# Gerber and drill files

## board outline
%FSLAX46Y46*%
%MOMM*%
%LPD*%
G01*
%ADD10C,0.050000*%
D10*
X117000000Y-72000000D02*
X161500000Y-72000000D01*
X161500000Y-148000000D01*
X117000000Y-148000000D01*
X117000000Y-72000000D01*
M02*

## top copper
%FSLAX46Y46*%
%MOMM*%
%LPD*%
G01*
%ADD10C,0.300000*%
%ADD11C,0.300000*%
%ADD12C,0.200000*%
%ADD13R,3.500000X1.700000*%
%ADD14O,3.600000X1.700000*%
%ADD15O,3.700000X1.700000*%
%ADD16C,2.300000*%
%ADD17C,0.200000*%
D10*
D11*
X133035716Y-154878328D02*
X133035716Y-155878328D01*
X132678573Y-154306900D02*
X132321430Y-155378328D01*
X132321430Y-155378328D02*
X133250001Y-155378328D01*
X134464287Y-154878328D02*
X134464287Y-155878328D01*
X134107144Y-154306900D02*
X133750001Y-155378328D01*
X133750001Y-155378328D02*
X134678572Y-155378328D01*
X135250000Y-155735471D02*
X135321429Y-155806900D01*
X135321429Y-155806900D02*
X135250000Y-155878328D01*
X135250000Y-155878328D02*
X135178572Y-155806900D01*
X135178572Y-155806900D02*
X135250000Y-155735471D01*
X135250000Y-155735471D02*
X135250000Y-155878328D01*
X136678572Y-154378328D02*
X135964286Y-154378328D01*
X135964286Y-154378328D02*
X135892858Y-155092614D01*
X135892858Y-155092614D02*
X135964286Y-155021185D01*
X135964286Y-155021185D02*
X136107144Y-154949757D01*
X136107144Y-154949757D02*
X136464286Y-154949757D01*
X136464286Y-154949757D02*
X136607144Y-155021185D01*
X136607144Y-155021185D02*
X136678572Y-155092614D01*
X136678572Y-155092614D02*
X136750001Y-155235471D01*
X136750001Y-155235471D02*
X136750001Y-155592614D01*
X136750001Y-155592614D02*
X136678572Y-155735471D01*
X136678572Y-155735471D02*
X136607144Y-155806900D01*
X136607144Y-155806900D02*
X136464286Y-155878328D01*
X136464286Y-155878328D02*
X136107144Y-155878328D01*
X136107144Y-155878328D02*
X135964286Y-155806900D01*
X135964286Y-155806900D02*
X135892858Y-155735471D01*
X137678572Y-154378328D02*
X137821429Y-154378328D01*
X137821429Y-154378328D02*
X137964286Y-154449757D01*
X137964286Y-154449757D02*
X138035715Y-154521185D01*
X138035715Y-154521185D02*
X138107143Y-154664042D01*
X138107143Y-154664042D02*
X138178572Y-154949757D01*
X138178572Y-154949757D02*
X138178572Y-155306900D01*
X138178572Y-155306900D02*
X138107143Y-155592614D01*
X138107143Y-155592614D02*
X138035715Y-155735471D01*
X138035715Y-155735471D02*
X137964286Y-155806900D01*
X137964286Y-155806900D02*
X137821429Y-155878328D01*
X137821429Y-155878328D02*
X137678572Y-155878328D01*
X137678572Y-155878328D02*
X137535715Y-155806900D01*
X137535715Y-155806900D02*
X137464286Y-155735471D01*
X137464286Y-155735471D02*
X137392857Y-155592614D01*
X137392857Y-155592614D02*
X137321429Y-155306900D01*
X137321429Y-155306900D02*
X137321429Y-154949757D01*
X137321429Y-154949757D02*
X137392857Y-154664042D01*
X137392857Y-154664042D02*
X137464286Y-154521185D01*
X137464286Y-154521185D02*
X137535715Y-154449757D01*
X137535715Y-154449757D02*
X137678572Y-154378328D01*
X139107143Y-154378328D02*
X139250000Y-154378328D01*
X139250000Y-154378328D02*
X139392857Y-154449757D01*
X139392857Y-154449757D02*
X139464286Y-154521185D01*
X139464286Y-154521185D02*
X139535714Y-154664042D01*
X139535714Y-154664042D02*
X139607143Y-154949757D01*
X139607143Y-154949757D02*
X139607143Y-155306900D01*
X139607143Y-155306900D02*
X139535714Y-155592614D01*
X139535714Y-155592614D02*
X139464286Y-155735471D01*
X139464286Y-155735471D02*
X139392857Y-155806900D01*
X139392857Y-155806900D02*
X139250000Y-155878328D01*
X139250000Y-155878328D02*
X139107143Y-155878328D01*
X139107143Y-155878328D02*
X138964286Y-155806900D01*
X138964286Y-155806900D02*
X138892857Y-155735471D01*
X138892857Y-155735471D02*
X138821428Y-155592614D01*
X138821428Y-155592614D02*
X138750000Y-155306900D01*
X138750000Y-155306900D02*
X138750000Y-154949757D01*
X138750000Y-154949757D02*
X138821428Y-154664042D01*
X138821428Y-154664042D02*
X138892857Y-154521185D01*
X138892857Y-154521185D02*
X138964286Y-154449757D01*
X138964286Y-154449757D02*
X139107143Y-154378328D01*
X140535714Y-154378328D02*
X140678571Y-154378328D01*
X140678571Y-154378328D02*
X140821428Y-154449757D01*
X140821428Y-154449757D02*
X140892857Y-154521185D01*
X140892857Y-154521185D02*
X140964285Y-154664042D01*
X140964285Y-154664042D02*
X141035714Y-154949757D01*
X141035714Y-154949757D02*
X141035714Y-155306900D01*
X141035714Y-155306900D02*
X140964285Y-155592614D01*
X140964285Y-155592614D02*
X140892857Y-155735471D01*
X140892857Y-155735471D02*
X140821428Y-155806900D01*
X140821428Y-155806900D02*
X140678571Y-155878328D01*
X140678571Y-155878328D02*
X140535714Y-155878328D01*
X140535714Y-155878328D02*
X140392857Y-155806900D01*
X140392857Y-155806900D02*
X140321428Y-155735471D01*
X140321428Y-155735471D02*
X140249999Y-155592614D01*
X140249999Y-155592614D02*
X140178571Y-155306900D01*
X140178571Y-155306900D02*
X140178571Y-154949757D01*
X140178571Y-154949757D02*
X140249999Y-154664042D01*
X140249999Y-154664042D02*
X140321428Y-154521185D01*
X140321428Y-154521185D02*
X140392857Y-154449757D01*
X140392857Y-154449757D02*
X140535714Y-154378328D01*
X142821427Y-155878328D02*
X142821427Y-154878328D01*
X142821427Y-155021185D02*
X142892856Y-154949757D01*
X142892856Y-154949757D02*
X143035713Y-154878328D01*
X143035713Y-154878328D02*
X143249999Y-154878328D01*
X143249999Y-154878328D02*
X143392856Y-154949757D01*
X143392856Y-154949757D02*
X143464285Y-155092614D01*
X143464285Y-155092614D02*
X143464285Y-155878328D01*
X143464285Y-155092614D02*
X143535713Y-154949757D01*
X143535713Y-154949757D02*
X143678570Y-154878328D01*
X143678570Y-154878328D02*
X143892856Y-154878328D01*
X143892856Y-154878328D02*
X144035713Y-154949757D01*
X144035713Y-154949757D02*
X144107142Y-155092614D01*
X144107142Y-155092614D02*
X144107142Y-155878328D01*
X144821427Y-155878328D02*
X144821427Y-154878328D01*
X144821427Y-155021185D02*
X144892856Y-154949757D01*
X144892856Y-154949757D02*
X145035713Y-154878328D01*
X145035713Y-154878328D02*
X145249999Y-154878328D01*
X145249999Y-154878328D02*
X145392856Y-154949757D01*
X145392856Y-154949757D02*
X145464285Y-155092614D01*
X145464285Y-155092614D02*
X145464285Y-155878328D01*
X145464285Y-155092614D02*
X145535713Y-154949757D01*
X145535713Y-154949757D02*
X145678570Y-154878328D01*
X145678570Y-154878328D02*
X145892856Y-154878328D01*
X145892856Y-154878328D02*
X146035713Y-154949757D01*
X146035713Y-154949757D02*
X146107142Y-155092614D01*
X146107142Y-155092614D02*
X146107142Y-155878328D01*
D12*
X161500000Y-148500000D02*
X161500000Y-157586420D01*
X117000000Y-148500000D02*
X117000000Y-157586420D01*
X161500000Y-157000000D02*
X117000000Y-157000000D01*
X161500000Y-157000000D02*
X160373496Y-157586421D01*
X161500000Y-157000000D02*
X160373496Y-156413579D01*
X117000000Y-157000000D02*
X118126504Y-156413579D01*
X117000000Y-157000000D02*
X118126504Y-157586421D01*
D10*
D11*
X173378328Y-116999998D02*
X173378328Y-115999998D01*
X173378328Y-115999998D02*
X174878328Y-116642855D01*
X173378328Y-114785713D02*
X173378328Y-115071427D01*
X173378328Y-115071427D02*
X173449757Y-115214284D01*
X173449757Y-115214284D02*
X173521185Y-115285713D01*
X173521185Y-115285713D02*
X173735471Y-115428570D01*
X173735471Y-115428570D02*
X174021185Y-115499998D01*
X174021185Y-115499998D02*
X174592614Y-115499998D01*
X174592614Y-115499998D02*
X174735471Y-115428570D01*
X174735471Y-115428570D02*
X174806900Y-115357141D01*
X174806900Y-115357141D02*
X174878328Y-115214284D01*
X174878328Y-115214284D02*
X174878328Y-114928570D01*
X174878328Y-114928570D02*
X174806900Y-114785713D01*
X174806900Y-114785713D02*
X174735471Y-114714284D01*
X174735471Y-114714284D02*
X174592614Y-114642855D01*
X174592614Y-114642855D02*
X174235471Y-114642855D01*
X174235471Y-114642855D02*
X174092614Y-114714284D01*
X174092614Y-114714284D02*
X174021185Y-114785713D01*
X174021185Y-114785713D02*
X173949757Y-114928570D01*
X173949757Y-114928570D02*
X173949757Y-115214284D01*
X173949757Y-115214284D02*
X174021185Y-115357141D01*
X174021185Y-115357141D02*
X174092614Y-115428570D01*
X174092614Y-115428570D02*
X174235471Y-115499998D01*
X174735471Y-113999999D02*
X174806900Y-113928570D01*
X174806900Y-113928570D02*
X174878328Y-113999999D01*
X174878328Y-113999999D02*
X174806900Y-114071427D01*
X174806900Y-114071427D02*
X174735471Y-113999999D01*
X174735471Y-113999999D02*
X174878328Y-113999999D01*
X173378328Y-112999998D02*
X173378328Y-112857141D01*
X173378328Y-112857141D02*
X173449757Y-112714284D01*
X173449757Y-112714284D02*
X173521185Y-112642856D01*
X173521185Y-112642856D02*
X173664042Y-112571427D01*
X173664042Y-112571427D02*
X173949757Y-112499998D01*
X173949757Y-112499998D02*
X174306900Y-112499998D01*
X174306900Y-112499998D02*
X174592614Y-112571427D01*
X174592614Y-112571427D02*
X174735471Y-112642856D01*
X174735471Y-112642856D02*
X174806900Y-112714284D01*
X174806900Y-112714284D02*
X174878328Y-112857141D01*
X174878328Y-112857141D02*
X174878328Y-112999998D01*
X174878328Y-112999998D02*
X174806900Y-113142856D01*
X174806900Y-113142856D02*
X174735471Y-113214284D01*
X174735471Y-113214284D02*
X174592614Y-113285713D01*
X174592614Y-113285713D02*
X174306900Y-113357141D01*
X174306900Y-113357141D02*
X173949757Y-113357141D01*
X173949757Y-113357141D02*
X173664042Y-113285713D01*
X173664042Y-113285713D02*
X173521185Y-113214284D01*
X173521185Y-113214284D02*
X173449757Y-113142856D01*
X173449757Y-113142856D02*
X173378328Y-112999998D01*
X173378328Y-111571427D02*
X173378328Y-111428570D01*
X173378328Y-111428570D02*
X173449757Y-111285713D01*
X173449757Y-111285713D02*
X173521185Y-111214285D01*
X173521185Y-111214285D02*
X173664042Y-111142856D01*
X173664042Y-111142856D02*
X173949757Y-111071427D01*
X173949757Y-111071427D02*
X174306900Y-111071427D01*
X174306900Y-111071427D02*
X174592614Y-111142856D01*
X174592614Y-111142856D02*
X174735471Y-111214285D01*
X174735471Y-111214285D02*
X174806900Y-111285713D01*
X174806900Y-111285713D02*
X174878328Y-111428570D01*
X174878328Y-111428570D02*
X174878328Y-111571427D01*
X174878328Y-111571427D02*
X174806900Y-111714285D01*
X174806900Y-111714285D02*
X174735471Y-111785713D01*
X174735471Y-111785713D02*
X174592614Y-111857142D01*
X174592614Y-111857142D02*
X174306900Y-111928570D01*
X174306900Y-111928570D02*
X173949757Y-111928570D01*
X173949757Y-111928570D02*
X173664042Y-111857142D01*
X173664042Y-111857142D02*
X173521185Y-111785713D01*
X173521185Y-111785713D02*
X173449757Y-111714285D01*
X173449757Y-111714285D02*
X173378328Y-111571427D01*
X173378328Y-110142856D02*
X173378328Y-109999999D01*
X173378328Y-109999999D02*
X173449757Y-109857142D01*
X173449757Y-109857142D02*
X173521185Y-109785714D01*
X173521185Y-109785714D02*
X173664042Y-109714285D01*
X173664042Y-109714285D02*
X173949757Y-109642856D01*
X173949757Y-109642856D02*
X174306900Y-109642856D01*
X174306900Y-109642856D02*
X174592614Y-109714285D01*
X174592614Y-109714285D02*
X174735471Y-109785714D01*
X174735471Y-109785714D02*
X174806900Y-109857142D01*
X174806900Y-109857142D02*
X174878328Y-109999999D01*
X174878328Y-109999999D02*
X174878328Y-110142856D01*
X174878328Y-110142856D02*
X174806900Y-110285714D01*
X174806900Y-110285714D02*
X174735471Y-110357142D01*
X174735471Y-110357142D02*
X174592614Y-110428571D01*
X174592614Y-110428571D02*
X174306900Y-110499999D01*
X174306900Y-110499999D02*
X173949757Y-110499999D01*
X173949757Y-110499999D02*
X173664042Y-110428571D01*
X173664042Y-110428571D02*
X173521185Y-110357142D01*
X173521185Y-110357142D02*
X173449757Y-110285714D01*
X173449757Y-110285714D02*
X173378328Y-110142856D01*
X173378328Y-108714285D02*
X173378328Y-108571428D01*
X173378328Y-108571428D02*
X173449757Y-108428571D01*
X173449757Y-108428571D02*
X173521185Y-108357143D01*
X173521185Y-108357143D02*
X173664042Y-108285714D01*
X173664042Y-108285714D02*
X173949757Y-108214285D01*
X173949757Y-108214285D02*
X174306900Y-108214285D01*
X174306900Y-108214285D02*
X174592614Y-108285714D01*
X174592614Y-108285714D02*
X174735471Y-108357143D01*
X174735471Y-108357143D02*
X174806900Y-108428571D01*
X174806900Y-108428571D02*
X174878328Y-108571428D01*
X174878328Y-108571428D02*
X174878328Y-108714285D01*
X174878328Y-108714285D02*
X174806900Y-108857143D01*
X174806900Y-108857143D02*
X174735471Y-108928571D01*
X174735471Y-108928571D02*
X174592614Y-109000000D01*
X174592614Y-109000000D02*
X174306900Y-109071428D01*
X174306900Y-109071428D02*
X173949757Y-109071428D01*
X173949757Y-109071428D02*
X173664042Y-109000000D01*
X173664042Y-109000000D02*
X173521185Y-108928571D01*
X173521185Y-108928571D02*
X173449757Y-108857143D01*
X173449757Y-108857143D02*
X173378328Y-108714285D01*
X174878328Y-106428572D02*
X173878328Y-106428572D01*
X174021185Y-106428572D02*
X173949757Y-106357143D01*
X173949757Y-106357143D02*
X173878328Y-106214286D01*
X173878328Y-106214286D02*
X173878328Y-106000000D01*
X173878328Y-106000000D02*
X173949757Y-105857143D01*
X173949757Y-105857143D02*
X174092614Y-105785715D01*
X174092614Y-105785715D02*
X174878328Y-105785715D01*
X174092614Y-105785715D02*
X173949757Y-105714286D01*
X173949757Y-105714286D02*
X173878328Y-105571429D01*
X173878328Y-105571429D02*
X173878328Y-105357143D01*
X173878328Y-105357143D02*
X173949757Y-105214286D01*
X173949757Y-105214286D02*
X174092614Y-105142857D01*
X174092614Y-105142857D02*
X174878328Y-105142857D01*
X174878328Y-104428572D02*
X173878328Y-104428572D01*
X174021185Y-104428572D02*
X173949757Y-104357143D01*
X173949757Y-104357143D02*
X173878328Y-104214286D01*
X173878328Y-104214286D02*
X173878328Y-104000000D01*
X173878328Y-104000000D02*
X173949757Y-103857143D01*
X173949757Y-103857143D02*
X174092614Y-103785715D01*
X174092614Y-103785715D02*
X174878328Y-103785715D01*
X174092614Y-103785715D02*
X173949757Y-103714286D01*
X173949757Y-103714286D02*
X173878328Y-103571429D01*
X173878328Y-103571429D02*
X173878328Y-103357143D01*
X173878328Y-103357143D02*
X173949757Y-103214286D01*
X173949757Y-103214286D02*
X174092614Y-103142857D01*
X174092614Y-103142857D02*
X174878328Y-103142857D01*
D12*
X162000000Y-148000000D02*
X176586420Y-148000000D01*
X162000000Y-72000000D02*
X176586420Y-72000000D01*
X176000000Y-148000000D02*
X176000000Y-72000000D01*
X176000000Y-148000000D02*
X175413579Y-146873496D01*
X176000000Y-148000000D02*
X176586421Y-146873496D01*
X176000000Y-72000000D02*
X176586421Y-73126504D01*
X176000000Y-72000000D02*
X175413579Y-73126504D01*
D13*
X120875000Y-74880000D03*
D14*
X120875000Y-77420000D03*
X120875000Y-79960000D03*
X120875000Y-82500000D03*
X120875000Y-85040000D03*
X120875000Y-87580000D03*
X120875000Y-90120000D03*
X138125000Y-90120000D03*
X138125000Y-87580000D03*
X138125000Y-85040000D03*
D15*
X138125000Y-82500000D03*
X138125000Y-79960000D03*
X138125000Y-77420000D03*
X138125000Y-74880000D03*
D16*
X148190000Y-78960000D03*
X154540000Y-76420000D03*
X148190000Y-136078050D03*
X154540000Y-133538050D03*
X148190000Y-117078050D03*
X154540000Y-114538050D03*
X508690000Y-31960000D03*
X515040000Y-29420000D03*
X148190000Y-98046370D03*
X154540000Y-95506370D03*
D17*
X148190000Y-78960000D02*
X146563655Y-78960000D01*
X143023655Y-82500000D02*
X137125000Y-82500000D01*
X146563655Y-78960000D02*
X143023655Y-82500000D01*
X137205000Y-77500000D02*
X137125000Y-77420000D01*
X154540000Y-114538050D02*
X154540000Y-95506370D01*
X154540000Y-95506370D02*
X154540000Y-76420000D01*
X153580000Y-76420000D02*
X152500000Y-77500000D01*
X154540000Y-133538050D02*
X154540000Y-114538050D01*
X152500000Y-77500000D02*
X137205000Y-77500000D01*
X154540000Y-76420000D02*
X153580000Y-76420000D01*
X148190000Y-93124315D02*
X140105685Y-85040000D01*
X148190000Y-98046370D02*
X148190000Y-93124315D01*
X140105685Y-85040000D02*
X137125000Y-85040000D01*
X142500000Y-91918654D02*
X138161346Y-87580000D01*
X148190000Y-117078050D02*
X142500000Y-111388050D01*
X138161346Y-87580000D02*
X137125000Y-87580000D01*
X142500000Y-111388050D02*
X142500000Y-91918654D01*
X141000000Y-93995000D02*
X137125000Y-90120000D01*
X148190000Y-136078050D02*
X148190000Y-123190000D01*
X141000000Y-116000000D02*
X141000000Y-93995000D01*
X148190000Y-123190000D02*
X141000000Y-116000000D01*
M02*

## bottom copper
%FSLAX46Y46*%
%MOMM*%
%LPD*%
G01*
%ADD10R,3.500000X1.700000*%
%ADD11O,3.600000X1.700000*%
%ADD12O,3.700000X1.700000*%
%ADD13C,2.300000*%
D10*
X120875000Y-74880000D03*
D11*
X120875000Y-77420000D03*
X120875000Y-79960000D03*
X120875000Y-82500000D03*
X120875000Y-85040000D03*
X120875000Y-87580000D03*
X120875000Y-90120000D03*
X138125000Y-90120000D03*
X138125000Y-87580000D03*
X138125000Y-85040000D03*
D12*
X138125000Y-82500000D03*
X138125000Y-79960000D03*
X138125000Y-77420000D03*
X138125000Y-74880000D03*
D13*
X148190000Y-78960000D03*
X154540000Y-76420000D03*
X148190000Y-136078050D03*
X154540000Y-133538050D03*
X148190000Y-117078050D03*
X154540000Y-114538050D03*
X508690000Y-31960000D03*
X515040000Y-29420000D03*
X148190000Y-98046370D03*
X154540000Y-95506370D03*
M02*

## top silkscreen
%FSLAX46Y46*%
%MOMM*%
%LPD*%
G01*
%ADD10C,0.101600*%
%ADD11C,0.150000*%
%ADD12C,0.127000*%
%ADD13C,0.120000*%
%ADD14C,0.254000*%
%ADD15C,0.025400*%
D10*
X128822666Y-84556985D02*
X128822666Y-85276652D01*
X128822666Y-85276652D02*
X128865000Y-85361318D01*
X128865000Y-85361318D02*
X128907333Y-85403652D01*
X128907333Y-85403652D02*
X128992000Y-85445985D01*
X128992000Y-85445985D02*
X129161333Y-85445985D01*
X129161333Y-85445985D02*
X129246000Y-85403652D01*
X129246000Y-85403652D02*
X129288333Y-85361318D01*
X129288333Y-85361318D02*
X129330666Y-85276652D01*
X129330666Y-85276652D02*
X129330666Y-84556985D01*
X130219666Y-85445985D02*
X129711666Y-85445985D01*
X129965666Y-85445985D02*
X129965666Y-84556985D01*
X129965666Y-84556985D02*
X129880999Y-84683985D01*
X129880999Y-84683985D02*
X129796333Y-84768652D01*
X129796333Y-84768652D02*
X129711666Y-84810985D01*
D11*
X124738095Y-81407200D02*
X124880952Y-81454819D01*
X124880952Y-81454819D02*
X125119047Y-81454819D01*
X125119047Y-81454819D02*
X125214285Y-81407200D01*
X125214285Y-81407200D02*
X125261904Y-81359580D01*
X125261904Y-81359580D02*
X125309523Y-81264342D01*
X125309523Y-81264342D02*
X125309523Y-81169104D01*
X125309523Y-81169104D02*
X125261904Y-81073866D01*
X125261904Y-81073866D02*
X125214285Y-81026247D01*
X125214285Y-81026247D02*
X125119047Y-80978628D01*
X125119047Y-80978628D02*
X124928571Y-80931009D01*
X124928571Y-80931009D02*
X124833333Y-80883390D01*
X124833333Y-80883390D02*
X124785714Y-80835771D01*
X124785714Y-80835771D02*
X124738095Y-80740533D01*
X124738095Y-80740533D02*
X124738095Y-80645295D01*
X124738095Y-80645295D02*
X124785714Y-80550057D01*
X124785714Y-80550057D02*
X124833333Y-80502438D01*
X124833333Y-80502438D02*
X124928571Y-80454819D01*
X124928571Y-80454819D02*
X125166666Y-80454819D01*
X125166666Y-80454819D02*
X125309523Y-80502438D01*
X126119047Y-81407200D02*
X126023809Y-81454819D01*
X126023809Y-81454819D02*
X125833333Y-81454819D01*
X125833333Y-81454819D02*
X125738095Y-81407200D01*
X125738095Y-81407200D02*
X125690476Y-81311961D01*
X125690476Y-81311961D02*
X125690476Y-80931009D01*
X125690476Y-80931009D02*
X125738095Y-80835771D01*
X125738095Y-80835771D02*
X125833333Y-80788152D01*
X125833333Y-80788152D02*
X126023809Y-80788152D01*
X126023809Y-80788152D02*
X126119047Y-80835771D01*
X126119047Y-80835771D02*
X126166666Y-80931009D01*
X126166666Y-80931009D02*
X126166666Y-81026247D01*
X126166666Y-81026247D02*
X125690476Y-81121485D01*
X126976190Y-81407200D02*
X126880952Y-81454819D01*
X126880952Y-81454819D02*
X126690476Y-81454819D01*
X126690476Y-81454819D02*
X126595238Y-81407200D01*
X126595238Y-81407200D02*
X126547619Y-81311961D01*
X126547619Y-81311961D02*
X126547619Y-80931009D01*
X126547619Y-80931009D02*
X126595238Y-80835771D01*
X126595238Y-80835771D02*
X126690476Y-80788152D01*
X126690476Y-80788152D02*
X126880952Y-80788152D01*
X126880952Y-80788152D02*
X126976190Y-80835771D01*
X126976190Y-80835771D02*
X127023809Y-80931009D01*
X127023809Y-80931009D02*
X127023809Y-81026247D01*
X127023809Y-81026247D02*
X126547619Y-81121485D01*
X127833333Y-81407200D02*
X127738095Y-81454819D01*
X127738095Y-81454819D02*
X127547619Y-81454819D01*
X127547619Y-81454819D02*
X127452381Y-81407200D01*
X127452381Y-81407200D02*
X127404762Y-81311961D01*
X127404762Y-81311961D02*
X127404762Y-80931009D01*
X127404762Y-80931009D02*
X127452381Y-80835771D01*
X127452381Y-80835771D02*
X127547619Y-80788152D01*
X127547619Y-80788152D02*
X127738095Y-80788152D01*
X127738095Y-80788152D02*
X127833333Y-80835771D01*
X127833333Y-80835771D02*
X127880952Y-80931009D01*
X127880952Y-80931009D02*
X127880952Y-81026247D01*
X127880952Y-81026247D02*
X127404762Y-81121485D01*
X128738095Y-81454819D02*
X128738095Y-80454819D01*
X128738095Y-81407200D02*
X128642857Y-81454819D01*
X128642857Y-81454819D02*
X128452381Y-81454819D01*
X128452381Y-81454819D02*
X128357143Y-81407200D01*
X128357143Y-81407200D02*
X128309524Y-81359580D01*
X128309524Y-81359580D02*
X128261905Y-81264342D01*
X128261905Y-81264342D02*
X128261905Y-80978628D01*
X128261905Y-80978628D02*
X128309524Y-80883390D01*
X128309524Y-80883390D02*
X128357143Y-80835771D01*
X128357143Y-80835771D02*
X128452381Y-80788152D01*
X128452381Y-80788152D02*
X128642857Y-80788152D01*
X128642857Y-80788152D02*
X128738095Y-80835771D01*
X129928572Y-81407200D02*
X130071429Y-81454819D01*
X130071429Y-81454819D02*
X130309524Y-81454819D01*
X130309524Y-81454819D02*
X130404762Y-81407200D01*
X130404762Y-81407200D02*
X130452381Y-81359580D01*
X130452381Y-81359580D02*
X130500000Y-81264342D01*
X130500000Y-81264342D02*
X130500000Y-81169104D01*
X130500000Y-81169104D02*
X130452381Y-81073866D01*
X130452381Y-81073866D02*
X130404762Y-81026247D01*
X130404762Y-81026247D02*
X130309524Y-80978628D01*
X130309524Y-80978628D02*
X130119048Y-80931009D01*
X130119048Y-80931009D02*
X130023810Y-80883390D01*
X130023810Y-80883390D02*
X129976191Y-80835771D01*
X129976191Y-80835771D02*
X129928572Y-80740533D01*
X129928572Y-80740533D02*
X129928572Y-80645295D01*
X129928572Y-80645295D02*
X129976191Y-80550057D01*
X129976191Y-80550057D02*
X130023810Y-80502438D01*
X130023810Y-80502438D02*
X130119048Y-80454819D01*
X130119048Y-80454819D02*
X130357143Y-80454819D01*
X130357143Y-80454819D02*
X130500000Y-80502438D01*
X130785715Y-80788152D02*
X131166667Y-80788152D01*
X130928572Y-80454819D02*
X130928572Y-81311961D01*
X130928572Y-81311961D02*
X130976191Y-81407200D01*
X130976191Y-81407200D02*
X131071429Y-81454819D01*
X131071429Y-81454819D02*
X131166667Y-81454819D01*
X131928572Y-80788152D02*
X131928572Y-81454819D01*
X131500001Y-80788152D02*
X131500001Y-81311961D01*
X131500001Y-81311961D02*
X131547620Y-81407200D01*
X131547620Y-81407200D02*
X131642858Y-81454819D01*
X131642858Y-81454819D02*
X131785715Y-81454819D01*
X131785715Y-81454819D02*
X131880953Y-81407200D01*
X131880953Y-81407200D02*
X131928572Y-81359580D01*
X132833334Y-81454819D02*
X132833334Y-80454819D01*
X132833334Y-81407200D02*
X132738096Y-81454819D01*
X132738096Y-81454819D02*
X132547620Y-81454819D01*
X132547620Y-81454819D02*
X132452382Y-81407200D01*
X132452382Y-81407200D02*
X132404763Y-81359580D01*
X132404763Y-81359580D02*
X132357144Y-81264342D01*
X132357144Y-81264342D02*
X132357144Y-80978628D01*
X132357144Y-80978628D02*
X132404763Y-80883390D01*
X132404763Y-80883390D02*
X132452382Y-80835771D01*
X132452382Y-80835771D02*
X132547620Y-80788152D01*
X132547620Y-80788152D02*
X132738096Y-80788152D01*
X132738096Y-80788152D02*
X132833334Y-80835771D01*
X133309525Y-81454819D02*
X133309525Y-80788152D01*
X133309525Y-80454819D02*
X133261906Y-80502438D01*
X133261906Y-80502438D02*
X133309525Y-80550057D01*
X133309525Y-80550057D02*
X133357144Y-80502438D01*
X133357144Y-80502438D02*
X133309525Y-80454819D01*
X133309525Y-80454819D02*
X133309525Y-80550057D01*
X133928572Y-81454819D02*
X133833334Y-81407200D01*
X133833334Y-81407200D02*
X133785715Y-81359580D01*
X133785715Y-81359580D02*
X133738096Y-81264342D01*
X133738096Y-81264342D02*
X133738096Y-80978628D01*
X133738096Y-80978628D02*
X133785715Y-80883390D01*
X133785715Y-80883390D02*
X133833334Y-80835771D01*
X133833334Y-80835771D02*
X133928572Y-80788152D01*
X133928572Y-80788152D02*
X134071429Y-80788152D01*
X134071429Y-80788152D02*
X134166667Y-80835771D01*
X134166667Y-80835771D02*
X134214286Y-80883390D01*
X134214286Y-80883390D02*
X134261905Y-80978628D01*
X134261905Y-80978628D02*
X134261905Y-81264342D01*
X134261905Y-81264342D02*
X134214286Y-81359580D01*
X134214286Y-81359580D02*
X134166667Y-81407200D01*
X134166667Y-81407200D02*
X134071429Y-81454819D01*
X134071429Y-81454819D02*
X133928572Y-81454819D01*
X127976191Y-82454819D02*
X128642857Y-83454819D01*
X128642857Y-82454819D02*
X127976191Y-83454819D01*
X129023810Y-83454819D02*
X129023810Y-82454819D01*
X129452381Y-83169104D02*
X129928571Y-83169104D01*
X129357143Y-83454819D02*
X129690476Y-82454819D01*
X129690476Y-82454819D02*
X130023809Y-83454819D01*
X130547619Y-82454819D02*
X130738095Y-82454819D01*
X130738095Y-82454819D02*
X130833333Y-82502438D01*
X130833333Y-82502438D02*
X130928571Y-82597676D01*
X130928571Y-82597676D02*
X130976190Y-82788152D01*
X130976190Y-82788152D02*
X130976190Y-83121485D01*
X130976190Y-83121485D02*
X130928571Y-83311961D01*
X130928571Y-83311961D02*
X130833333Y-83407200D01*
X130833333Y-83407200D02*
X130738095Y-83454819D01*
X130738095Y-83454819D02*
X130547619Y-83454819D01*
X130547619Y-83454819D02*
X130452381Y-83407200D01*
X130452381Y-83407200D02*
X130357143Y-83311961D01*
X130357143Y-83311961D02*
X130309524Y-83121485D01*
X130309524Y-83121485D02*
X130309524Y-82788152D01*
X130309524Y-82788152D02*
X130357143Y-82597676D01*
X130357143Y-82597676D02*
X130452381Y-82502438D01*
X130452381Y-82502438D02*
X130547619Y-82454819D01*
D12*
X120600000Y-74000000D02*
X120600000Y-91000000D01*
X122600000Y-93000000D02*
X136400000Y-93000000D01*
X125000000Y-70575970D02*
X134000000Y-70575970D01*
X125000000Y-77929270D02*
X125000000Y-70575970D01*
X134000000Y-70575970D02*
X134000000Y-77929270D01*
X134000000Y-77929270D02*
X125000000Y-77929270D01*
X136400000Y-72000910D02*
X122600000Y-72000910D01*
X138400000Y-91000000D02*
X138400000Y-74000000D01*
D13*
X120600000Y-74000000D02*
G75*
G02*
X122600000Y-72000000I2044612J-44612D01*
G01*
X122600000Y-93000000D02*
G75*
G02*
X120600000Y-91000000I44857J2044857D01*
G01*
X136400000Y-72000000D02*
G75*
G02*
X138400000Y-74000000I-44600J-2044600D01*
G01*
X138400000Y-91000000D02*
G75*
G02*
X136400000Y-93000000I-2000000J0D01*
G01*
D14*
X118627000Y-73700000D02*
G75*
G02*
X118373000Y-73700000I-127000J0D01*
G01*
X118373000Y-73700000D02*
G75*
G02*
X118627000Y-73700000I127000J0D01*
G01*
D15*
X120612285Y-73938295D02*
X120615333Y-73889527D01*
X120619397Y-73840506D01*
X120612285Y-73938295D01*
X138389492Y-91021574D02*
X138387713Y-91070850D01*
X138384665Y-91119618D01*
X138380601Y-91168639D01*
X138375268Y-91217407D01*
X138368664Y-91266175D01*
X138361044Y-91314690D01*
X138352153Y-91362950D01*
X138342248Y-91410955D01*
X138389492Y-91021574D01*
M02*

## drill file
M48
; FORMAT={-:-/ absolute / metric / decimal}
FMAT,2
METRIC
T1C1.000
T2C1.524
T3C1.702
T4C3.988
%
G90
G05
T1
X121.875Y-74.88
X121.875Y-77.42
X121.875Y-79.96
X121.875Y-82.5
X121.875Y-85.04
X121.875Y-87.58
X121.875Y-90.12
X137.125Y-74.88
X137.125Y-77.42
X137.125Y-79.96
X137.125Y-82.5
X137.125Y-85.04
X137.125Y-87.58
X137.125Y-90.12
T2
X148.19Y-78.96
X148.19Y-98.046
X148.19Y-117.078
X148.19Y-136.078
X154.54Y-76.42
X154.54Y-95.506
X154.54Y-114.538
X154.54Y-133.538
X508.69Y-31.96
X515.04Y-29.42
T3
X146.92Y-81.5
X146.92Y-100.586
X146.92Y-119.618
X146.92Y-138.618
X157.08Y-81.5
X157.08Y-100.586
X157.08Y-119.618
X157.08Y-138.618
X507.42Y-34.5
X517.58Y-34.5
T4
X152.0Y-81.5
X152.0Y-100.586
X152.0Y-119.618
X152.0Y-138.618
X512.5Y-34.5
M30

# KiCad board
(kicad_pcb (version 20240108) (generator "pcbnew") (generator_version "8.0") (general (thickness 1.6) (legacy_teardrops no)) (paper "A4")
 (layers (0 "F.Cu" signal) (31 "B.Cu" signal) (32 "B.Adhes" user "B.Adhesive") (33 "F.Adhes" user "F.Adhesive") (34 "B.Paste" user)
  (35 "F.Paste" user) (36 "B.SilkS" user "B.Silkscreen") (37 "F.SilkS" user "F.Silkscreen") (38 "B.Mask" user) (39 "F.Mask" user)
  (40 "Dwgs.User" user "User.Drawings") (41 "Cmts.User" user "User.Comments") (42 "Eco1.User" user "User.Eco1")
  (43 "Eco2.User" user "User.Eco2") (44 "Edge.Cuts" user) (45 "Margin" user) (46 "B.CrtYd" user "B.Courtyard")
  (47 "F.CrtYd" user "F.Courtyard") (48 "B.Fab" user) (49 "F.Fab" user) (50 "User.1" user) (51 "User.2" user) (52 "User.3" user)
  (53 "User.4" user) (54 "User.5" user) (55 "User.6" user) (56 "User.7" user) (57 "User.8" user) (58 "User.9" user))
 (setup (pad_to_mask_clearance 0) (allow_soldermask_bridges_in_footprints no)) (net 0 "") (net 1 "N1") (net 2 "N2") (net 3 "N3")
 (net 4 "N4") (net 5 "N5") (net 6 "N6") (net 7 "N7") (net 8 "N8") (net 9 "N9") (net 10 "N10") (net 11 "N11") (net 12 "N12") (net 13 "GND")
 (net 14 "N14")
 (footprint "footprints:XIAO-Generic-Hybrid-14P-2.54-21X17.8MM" (layer "F.Cu") (at 129.5 82.5)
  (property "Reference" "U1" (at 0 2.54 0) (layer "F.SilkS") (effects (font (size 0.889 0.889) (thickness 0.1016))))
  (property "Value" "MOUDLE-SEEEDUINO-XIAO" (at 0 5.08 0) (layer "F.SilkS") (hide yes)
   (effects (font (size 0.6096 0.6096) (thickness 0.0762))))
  (fp_line (start -8.9 -8.5) (end -8.9 8.5) (stroke (width 0.127) (type solid)) (layer "F.SilkS"))
  (fp_line (start -6.9 10.5) (end 6.9 10.5) (stroke (width 0.127) (type solid)) (layer "F.SilkS"))
  (fp_line (start -4.5 -11.92403) (end 4.5 -11.92403) (stroke (width 0.127) (type solid)) (layer "F.SilkS"))
  (fp_line (start -4.5 -4.57073) (end -4.5 -11.92403) (stroke (width 0.127) (type solid)) (layer "F.SilkS"))
  (fp_line (start 4.5 -11.92403) (end 4.5 -4.57073) (stroke (width 0.127) (type solid)) (layer "F.SilkS"))
  (fp_line (start 4.5 -4.57073) (end -4.5 -4.57073) (stroke (width 0.127) (type solid)) (layer "F.SilkS"))
  (fp_line (start 6.9 -10.49909) (end -6.9 -10.49909) (stroke (width 0.127) (type solid)) (layer "F.SilkS"))
  (fp_line (start 8.9 8.5) (end 8.9 -8.5) (stroke (width 0.127) (type solid)) (layer "F.SilkS"))
  (fp_arc (start -8.9 -8.5) (mid -8.301491 -9.901491) (end -6.9 -10.5) (stroke (width 0.12) (type solid)) (layer "F.SilkS"))
  (fp_arc (start -6.9 10.5) (mid -8.301423 9.901423) (end -8.9 8.5) (stroke (width 0.12) (type solid)) (layer "F.SilkS"))
  (fp_arc (start 6.9 -10.5) (mid 8.301492 -9.901492) (end 8.9 -8.5) (stroke (width 0.12) (type solid)) (layer "F.SilkS"))
  (fp_arc (start 8.9 8.5) (mid 8.314214 9.914214) (end 6.9 10.5) (stroke (width 0.12) (type solid)) (layer "F.SilkS"))
  (fp_circle (center -11 -8.8) (end -11 -9.054) (stroke (width 0) (type solid)) (fill solid) (layer "F.SilkS"))
  (fp_poly
   (pts (xy -8.887715 -8.561705) (xy -8.884667 -8.610473) (xy -8.880603 -8.659494)) (stroke (width 0.0254) (type solid)) (fill none)
   (layer "F.SilkS"))
  (fp_poly
   (pts (xy 8.889492 8.521574) (xy 8.887713 8.57085) (xy 8.884665 8.619618) (xy 8.880601 8.668639) (xy 8.875268 8.717407)
    (xy 8.868664 8.766175) (xy 8.861044 8.81469) (xy 8.852153 8.86295) (xy 8.842248 8.910955))
   (stroke (width 0.0254) (type solid)) (fill none) (layer "F.SilkS"))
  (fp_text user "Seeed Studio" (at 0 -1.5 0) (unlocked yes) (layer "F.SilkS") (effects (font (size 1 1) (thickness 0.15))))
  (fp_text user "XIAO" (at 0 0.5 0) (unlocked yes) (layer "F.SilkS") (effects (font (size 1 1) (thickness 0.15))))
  (pad "1" thru_hole rect (at -7.625 -7.62) (size 3.5 1.7) (drill 1 (offset -1 0)) (layers "*.Cu" "*.Mask") (remove_unused_layers no)
   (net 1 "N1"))
  (pad "2" thru_hole oval (at -7.625 -5.08) (size 3.6 1.7) (drill 1 (offset -1 0)) (layers "*.Cu" "*.Mask") (remove_unused_layers no)
   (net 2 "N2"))
  (pad "3" thru_hole oval (at -7.625 -2.54) (size 3.6 1.7) (drill 1 (offset -1 0)) (layers "*.Cu" "*.Mask") (remove_unused_layers no)
   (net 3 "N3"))
  (pad "4" thru_hole oval (at -7.625 0) (size 3.6 1.7) (drill 1 (offset -1 0)) (layers "*.Cu" "*.Mask") (remove_unused_layers no)
   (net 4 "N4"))
  (pad "5" thru_hole oval (at -7.625 2.54) (size 3.6 1.7) (drill 1 (offset -1 0)) (layers "*.Cu" "*.Mask") (remove_unused_layers no)
   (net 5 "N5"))
  (pad "6" thru_hole oval (at -7.625 5.08 180) (size 3.6 1.7) (drill 1 (offset 1 0)) (layers "*.Cu" "*.Mask") (remove_unused_layers no)
   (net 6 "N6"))
  (pad "7" thru_hole oval (at -7.625 7.62) (size 3.6 1.7) (drill 1 (offset -1 0)) (layers "*.Cu" "*.Mask") (remove_unused_layers no)
   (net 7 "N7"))
  (pad "8" thru_hole oval (at 7.625 7.62) (size 3.6 1.7) (drill 1 (offset 1 0)) (layers "*.Cu" "*.Mask") (remove_unused_layers no)
   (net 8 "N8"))
  (pad "9" thru_hole oval (at 7.625 5.08) (size 3.6 1.7) (drill 1 (offset 1 0)) (layers "*.Cu" "*.Mask") (remove_unused_layers no)
   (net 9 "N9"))
  (pad "10" thru_hole oval (at 7.625 2.54) (size 3.6 1.7) (drill 1 (offset 1 0)) (layers "*.Cu" "*.Mask") (remove_unused_layers no)
   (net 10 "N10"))
  (pad "11" thru_hole oval (at 7.625 0) (size 3.7 1.7) (drill 1 (offset 1 0)) (layers "*.Cu" "*.Mask") (remove_unused_layers no)
   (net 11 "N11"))
  (pad "12" thru_hole oval (at 7.625 -2.54) (size 3.7 1.7) (drill 1 (offset 1 0)) (layers "*.Cu" "*.Mask") (remove_unused_layers no)
   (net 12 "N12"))
  (pad "13" thru_hole oval (at 7.625 -5.08) (size 3.7 1.7) (drill 1 (offset 1 0)) (layers "*.Cu" "*.Mask") (remove_unused_layers no)
   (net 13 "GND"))
  (pad "14" thru_hole oval (at 7.625 -7.62) (size 3.7 1.7) (drill 1 (offset 1 0)) (layers "*.Cu" "*.Mask") (remove_unused_layers no)
   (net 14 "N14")))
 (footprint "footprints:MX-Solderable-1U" (layer "F.Cu") (at 152 81.5)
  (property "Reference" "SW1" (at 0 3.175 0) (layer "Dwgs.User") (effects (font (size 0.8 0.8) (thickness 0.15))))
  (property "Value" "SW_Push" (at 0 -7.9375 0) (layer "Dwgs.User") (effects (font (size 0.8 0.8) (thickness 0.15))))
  (pad "" np_thru_hole circle (at -5.08 0 48.099) (size 1.7018 1.7018) (drill 1.7018) (layers "F&B.Cu" "*.Mask"))
  (pad "" np_thru_hole circle (at 0 0) (size 3.9878 3.9878) (drill 3.9878) (layers "*.Cu" "*.Mask"))
  (pad "" np_thru_hole circle (at 5.08 0 48.099) (size 1.7018 1.7018) (drill 1.7018) (layers "F&B.Cu" "*.Mask"))
  (pad "1" thru_hole circle (at -3.81 -2.54) (size 2.3 2.3) (drill 1.524) (layers "*.Cu" "B.Mask") (remove_unused_layers no) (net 11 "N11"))
  (pad "2" thru_hole circle (at 2.54 -5.08) (size 2.3 2.3) (drill 1.524) (layers "*.Cu" "B.Mask") (remove_unused_layers no) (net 13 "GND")))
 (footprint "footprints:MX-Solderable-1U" (layer "F.Cu") (at 152 138.61805)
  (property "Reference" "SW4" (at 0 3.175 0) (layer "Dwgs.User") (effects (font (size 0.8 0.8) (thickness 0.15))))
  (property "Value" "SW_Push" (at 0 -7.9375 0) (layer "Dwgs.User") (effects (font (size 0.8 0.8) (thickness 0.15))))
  (pad "" np_thru_hole circle (at -5.08 0 48.099) (size 1.7018 1.7018) (drill 1.7018) (layers "F&B.Cu" "*.Mask"))
  (pad "" np_thru_hole circle (at 0 0) (size 3.9878 3.9878) (drill 3.9878) (layers "*.Cu" "*.Mask"))
  (pad "" np_thru_hole circle (at 5.08 0 48.099) (size 1.7018 1.7018) (drill 1.7018) (layers "F&B.Cu" "*.Mask"))
  (pad "1" thru_hole circle (at -3.81 -2.54) (size 2.3 2.3) (drill 1.524) (layers "*.Cu" "B.Mask") (remove_unused_layers no) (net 8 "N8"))
  (pad "2" thru_hole circle (at 2.54 -5.08) (size 2.3 2.3) (drill 1.524) (layers "*.Cu" "B.Mask") (remove_unused_layers no) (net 13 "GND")))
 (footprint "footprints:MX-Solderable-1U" (layer "F.Cu") (at 152 119.61805)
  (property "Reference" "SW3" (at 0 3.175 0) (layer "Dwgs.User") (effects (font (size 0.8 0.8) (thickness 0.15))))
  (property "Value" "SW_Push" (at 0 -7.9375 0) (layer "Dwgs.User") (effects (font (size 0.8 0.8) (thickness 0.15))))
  (pad "" np_thru_hole circle (at -5.08 0 48.099) (size 1.7018 1.7018) (drill 1.7018) (layers "F&B.Cu" "*.Mask"))
  (pad "" np_thru_hole circle (at 0 0) (size 3.9878 3.9878) (drill 3.9878) (layers "*.Cu" "*.Mask"))
  (pad "" np_thru_hole circle (at 5.08 0 48.099) (size 1.7018 1.7018) (drill 1.7018) (layers "F&B.Cu" "*.Mask"))
  (pad "1" thru_hole circle (at -3.81 -2.54) (size 2.3 2.3) (drill 1.524) (layers "*.Cu" "B.Mask") (remove_unused_layers no) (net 9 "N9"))
  (pad "2" thru_hole circle (at 2.54 -5.08) (size 2.3 2.3) (drill 1.524) (layers "*.Cu" "B.Mask") (remove_unused_layers no) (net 13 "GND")))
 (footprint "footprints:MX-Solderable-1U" (layer "F.Cu") (at 512.5 34.5)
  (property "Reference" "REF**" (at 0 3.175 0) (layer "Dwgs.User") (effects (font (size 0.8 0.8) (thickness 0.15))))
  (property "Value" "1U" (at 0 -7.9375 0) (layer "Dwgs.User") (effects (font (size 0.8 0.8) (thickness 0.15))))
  (pad "" np_thru_hole circle (at -5.08 0 48.099) (size 1.7018 1.7018) (drill 1.7018) (layers "F&B.Cu" "*.Mask"))
  (pad "" np_thru_hole circle (at 0 0) (size 3.9878 3.9878) (drill 3.9878) (layers "*.Cu" "*.Mask"))
  (pad "" np_thru_hole circle (at 5.08 0 48.099) (size 1.7018 1.7018) (drill 1.7018) (layers "F&B.Cu" "*.Mask"))
  (pad "1" thru_hole circle (at -3.81 -2.54) (size 2.3 2.3) (drill 1.524) (layers "*.Cu" "B.Mask") (remove_unused_layers no))
  (pad "2" thru_hole circle (at 2.54 -5.08) (size 2.3 2.3) (drill 1.524) (layers "*.Cu" "B.Mask") (remove_unused_layers no)))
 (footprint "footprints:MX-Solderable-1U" (layer "F.Cu") (at 152 100.58637)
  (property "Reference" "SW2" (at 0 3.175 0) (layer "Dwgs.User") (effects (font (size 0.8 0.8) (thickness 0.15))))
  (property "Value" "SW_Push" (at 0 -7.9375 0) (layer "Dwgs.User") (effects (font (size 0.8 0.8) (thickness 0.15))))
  (pad "" np_thru_hole circle (at -5.08 0 48.099) (size 1.7018 1.7018) (drill 1.7018) (layers "F&B.Cu" "*.Mask"))
  (pad "" np_thru_hole circle (at 0 0) (size 3.9878 3.9878) (drill 3.9878) (layers "*.Cu" "*.Mask"))
  (pad "" np_thru_hole circle (at 5.08 0 48.099) (size 1.7018 1.7018) (drill 1.7018) (layers "F&B.Cu" "*.Mask"))
  (pad "1" thru_hole circle (at -3.81 -2.54) (size 2.3 2.3) (drill 1.524) (layers "*.Cu" "B.Mask") (remove_unused_layers no) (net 10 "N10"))
  (pad "2" thru_hole circle (at 2.54 -5.08) (size 2.3 2.3) (drill 1.524) (layers "*.Cu" "B.Mask") (remove_unused_layers no) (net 13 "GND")))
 (gr_rect (start 117 72) (end 161.5 148) (stroke (width 0.05) (type default)) (fill none) (layer "Edge.Cuts"))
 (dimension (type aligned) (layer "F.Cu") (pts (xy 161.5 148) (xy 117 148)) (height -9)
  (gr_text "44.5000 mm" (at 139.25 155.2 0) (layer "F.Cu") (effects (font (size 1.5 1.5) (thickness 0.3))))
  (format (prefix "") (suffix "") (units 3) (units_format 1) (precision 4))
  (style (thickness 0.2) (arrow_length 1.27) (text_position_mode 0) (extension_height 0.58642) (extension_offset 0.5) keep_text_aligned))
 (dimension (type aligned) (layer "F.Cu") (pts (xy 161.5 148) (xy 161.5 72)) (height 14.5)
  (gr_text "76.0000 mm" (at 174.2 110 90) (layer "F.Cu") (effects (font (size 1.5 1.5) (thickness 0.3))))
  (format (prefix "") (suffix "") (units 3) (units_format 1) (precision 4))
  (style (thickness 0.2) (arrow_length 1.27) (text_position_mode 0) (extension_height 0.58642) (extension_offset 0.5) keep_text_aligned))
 (segment (start 148.19 78.96) (end 146.563655 78.96) (width 0.2) (layer "F.Cu") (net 11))
 (segment (start 143.023655 82.5) (end 137.125 82.5) (width 0.2) (layer "F.Cu") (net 11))
 (segment (start 146.563655 78.96) (end 143.023655 82.5) (width 0.2) (layer "F.Cu") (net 11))
 (segment (start 137.205 77.5) (end 137.125 77.42) (width 0.2) (layer "F.Cu") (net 13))
 (segment (start 154.54 114.53805) (end 154.54 95.50637) (width 0.2) (layer "F.Cu") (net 13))
 (segment (start 154.54 95.50637) (end 154.54 76.42) (width 0.2) (layer "F.Cu") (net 13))
 (segment (start 153.58 76.42) (end 152.5 77.5) (width 0.2) (layer "F.Cu") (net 13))
 (segment (start 154.54 133.53805) (end 154.54 114.53805) (width 0.2) (layer "F.Cu") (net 13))
 (segment (start 152.5 77.5) (end 137.205 77.5) (width 0.2) (layer "F.Cu") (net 13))
 (segment (start 154.54 76.42) (end 153.58 76.42) (width 0.2) (layer "F.Cu") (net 13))
 (segment (start 148.19 93.124315) (end 140.105685 85.04) (width 0.2) (layer "F.Cu") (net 10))
 (segment (start 148.19 98.04637) (end 148.19 93.124315) (width 0.2) (layer "F.Cu") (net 10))
 (segment (start 140.105685 85.04) (end 137.125 85.04) (width 0.2) (layer "F.Cu") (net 10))
 (segment (start 142.5 91.918654) (end 138.161346 87.58) (width 0.2) (layer "F.Cu") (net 9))
 (segment (start 148.19 117.07805) (end 142.5 111.38805) (width 0.2) (layer "F.Cu") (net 9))
 (segment (start 138.161346 87.58) (end 137.125 87.58) (width 0.2) (layer "F.Cu") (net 9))
 (segment (start 142.5 111.38805) (end 142.5 91.918654) (width 0.2) (layer "F.Cu") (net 9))
 (segment (start 141 93.995) (end 137.125 90.12) (width 0.2) (layer "F.Cu") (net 8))
 (segment (start 148.19 136.07805) (end 148.19 123.19) (width 0.2) (layer "F.Cu") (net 8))
 (segment (start 141 116) (end 141 93.995) (width 0.2) (layer "F.Cu") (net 8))
 (segment (start 148.19 123.19) (end 141 116) (width 0.2) (layer "F.Cu") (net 8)))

